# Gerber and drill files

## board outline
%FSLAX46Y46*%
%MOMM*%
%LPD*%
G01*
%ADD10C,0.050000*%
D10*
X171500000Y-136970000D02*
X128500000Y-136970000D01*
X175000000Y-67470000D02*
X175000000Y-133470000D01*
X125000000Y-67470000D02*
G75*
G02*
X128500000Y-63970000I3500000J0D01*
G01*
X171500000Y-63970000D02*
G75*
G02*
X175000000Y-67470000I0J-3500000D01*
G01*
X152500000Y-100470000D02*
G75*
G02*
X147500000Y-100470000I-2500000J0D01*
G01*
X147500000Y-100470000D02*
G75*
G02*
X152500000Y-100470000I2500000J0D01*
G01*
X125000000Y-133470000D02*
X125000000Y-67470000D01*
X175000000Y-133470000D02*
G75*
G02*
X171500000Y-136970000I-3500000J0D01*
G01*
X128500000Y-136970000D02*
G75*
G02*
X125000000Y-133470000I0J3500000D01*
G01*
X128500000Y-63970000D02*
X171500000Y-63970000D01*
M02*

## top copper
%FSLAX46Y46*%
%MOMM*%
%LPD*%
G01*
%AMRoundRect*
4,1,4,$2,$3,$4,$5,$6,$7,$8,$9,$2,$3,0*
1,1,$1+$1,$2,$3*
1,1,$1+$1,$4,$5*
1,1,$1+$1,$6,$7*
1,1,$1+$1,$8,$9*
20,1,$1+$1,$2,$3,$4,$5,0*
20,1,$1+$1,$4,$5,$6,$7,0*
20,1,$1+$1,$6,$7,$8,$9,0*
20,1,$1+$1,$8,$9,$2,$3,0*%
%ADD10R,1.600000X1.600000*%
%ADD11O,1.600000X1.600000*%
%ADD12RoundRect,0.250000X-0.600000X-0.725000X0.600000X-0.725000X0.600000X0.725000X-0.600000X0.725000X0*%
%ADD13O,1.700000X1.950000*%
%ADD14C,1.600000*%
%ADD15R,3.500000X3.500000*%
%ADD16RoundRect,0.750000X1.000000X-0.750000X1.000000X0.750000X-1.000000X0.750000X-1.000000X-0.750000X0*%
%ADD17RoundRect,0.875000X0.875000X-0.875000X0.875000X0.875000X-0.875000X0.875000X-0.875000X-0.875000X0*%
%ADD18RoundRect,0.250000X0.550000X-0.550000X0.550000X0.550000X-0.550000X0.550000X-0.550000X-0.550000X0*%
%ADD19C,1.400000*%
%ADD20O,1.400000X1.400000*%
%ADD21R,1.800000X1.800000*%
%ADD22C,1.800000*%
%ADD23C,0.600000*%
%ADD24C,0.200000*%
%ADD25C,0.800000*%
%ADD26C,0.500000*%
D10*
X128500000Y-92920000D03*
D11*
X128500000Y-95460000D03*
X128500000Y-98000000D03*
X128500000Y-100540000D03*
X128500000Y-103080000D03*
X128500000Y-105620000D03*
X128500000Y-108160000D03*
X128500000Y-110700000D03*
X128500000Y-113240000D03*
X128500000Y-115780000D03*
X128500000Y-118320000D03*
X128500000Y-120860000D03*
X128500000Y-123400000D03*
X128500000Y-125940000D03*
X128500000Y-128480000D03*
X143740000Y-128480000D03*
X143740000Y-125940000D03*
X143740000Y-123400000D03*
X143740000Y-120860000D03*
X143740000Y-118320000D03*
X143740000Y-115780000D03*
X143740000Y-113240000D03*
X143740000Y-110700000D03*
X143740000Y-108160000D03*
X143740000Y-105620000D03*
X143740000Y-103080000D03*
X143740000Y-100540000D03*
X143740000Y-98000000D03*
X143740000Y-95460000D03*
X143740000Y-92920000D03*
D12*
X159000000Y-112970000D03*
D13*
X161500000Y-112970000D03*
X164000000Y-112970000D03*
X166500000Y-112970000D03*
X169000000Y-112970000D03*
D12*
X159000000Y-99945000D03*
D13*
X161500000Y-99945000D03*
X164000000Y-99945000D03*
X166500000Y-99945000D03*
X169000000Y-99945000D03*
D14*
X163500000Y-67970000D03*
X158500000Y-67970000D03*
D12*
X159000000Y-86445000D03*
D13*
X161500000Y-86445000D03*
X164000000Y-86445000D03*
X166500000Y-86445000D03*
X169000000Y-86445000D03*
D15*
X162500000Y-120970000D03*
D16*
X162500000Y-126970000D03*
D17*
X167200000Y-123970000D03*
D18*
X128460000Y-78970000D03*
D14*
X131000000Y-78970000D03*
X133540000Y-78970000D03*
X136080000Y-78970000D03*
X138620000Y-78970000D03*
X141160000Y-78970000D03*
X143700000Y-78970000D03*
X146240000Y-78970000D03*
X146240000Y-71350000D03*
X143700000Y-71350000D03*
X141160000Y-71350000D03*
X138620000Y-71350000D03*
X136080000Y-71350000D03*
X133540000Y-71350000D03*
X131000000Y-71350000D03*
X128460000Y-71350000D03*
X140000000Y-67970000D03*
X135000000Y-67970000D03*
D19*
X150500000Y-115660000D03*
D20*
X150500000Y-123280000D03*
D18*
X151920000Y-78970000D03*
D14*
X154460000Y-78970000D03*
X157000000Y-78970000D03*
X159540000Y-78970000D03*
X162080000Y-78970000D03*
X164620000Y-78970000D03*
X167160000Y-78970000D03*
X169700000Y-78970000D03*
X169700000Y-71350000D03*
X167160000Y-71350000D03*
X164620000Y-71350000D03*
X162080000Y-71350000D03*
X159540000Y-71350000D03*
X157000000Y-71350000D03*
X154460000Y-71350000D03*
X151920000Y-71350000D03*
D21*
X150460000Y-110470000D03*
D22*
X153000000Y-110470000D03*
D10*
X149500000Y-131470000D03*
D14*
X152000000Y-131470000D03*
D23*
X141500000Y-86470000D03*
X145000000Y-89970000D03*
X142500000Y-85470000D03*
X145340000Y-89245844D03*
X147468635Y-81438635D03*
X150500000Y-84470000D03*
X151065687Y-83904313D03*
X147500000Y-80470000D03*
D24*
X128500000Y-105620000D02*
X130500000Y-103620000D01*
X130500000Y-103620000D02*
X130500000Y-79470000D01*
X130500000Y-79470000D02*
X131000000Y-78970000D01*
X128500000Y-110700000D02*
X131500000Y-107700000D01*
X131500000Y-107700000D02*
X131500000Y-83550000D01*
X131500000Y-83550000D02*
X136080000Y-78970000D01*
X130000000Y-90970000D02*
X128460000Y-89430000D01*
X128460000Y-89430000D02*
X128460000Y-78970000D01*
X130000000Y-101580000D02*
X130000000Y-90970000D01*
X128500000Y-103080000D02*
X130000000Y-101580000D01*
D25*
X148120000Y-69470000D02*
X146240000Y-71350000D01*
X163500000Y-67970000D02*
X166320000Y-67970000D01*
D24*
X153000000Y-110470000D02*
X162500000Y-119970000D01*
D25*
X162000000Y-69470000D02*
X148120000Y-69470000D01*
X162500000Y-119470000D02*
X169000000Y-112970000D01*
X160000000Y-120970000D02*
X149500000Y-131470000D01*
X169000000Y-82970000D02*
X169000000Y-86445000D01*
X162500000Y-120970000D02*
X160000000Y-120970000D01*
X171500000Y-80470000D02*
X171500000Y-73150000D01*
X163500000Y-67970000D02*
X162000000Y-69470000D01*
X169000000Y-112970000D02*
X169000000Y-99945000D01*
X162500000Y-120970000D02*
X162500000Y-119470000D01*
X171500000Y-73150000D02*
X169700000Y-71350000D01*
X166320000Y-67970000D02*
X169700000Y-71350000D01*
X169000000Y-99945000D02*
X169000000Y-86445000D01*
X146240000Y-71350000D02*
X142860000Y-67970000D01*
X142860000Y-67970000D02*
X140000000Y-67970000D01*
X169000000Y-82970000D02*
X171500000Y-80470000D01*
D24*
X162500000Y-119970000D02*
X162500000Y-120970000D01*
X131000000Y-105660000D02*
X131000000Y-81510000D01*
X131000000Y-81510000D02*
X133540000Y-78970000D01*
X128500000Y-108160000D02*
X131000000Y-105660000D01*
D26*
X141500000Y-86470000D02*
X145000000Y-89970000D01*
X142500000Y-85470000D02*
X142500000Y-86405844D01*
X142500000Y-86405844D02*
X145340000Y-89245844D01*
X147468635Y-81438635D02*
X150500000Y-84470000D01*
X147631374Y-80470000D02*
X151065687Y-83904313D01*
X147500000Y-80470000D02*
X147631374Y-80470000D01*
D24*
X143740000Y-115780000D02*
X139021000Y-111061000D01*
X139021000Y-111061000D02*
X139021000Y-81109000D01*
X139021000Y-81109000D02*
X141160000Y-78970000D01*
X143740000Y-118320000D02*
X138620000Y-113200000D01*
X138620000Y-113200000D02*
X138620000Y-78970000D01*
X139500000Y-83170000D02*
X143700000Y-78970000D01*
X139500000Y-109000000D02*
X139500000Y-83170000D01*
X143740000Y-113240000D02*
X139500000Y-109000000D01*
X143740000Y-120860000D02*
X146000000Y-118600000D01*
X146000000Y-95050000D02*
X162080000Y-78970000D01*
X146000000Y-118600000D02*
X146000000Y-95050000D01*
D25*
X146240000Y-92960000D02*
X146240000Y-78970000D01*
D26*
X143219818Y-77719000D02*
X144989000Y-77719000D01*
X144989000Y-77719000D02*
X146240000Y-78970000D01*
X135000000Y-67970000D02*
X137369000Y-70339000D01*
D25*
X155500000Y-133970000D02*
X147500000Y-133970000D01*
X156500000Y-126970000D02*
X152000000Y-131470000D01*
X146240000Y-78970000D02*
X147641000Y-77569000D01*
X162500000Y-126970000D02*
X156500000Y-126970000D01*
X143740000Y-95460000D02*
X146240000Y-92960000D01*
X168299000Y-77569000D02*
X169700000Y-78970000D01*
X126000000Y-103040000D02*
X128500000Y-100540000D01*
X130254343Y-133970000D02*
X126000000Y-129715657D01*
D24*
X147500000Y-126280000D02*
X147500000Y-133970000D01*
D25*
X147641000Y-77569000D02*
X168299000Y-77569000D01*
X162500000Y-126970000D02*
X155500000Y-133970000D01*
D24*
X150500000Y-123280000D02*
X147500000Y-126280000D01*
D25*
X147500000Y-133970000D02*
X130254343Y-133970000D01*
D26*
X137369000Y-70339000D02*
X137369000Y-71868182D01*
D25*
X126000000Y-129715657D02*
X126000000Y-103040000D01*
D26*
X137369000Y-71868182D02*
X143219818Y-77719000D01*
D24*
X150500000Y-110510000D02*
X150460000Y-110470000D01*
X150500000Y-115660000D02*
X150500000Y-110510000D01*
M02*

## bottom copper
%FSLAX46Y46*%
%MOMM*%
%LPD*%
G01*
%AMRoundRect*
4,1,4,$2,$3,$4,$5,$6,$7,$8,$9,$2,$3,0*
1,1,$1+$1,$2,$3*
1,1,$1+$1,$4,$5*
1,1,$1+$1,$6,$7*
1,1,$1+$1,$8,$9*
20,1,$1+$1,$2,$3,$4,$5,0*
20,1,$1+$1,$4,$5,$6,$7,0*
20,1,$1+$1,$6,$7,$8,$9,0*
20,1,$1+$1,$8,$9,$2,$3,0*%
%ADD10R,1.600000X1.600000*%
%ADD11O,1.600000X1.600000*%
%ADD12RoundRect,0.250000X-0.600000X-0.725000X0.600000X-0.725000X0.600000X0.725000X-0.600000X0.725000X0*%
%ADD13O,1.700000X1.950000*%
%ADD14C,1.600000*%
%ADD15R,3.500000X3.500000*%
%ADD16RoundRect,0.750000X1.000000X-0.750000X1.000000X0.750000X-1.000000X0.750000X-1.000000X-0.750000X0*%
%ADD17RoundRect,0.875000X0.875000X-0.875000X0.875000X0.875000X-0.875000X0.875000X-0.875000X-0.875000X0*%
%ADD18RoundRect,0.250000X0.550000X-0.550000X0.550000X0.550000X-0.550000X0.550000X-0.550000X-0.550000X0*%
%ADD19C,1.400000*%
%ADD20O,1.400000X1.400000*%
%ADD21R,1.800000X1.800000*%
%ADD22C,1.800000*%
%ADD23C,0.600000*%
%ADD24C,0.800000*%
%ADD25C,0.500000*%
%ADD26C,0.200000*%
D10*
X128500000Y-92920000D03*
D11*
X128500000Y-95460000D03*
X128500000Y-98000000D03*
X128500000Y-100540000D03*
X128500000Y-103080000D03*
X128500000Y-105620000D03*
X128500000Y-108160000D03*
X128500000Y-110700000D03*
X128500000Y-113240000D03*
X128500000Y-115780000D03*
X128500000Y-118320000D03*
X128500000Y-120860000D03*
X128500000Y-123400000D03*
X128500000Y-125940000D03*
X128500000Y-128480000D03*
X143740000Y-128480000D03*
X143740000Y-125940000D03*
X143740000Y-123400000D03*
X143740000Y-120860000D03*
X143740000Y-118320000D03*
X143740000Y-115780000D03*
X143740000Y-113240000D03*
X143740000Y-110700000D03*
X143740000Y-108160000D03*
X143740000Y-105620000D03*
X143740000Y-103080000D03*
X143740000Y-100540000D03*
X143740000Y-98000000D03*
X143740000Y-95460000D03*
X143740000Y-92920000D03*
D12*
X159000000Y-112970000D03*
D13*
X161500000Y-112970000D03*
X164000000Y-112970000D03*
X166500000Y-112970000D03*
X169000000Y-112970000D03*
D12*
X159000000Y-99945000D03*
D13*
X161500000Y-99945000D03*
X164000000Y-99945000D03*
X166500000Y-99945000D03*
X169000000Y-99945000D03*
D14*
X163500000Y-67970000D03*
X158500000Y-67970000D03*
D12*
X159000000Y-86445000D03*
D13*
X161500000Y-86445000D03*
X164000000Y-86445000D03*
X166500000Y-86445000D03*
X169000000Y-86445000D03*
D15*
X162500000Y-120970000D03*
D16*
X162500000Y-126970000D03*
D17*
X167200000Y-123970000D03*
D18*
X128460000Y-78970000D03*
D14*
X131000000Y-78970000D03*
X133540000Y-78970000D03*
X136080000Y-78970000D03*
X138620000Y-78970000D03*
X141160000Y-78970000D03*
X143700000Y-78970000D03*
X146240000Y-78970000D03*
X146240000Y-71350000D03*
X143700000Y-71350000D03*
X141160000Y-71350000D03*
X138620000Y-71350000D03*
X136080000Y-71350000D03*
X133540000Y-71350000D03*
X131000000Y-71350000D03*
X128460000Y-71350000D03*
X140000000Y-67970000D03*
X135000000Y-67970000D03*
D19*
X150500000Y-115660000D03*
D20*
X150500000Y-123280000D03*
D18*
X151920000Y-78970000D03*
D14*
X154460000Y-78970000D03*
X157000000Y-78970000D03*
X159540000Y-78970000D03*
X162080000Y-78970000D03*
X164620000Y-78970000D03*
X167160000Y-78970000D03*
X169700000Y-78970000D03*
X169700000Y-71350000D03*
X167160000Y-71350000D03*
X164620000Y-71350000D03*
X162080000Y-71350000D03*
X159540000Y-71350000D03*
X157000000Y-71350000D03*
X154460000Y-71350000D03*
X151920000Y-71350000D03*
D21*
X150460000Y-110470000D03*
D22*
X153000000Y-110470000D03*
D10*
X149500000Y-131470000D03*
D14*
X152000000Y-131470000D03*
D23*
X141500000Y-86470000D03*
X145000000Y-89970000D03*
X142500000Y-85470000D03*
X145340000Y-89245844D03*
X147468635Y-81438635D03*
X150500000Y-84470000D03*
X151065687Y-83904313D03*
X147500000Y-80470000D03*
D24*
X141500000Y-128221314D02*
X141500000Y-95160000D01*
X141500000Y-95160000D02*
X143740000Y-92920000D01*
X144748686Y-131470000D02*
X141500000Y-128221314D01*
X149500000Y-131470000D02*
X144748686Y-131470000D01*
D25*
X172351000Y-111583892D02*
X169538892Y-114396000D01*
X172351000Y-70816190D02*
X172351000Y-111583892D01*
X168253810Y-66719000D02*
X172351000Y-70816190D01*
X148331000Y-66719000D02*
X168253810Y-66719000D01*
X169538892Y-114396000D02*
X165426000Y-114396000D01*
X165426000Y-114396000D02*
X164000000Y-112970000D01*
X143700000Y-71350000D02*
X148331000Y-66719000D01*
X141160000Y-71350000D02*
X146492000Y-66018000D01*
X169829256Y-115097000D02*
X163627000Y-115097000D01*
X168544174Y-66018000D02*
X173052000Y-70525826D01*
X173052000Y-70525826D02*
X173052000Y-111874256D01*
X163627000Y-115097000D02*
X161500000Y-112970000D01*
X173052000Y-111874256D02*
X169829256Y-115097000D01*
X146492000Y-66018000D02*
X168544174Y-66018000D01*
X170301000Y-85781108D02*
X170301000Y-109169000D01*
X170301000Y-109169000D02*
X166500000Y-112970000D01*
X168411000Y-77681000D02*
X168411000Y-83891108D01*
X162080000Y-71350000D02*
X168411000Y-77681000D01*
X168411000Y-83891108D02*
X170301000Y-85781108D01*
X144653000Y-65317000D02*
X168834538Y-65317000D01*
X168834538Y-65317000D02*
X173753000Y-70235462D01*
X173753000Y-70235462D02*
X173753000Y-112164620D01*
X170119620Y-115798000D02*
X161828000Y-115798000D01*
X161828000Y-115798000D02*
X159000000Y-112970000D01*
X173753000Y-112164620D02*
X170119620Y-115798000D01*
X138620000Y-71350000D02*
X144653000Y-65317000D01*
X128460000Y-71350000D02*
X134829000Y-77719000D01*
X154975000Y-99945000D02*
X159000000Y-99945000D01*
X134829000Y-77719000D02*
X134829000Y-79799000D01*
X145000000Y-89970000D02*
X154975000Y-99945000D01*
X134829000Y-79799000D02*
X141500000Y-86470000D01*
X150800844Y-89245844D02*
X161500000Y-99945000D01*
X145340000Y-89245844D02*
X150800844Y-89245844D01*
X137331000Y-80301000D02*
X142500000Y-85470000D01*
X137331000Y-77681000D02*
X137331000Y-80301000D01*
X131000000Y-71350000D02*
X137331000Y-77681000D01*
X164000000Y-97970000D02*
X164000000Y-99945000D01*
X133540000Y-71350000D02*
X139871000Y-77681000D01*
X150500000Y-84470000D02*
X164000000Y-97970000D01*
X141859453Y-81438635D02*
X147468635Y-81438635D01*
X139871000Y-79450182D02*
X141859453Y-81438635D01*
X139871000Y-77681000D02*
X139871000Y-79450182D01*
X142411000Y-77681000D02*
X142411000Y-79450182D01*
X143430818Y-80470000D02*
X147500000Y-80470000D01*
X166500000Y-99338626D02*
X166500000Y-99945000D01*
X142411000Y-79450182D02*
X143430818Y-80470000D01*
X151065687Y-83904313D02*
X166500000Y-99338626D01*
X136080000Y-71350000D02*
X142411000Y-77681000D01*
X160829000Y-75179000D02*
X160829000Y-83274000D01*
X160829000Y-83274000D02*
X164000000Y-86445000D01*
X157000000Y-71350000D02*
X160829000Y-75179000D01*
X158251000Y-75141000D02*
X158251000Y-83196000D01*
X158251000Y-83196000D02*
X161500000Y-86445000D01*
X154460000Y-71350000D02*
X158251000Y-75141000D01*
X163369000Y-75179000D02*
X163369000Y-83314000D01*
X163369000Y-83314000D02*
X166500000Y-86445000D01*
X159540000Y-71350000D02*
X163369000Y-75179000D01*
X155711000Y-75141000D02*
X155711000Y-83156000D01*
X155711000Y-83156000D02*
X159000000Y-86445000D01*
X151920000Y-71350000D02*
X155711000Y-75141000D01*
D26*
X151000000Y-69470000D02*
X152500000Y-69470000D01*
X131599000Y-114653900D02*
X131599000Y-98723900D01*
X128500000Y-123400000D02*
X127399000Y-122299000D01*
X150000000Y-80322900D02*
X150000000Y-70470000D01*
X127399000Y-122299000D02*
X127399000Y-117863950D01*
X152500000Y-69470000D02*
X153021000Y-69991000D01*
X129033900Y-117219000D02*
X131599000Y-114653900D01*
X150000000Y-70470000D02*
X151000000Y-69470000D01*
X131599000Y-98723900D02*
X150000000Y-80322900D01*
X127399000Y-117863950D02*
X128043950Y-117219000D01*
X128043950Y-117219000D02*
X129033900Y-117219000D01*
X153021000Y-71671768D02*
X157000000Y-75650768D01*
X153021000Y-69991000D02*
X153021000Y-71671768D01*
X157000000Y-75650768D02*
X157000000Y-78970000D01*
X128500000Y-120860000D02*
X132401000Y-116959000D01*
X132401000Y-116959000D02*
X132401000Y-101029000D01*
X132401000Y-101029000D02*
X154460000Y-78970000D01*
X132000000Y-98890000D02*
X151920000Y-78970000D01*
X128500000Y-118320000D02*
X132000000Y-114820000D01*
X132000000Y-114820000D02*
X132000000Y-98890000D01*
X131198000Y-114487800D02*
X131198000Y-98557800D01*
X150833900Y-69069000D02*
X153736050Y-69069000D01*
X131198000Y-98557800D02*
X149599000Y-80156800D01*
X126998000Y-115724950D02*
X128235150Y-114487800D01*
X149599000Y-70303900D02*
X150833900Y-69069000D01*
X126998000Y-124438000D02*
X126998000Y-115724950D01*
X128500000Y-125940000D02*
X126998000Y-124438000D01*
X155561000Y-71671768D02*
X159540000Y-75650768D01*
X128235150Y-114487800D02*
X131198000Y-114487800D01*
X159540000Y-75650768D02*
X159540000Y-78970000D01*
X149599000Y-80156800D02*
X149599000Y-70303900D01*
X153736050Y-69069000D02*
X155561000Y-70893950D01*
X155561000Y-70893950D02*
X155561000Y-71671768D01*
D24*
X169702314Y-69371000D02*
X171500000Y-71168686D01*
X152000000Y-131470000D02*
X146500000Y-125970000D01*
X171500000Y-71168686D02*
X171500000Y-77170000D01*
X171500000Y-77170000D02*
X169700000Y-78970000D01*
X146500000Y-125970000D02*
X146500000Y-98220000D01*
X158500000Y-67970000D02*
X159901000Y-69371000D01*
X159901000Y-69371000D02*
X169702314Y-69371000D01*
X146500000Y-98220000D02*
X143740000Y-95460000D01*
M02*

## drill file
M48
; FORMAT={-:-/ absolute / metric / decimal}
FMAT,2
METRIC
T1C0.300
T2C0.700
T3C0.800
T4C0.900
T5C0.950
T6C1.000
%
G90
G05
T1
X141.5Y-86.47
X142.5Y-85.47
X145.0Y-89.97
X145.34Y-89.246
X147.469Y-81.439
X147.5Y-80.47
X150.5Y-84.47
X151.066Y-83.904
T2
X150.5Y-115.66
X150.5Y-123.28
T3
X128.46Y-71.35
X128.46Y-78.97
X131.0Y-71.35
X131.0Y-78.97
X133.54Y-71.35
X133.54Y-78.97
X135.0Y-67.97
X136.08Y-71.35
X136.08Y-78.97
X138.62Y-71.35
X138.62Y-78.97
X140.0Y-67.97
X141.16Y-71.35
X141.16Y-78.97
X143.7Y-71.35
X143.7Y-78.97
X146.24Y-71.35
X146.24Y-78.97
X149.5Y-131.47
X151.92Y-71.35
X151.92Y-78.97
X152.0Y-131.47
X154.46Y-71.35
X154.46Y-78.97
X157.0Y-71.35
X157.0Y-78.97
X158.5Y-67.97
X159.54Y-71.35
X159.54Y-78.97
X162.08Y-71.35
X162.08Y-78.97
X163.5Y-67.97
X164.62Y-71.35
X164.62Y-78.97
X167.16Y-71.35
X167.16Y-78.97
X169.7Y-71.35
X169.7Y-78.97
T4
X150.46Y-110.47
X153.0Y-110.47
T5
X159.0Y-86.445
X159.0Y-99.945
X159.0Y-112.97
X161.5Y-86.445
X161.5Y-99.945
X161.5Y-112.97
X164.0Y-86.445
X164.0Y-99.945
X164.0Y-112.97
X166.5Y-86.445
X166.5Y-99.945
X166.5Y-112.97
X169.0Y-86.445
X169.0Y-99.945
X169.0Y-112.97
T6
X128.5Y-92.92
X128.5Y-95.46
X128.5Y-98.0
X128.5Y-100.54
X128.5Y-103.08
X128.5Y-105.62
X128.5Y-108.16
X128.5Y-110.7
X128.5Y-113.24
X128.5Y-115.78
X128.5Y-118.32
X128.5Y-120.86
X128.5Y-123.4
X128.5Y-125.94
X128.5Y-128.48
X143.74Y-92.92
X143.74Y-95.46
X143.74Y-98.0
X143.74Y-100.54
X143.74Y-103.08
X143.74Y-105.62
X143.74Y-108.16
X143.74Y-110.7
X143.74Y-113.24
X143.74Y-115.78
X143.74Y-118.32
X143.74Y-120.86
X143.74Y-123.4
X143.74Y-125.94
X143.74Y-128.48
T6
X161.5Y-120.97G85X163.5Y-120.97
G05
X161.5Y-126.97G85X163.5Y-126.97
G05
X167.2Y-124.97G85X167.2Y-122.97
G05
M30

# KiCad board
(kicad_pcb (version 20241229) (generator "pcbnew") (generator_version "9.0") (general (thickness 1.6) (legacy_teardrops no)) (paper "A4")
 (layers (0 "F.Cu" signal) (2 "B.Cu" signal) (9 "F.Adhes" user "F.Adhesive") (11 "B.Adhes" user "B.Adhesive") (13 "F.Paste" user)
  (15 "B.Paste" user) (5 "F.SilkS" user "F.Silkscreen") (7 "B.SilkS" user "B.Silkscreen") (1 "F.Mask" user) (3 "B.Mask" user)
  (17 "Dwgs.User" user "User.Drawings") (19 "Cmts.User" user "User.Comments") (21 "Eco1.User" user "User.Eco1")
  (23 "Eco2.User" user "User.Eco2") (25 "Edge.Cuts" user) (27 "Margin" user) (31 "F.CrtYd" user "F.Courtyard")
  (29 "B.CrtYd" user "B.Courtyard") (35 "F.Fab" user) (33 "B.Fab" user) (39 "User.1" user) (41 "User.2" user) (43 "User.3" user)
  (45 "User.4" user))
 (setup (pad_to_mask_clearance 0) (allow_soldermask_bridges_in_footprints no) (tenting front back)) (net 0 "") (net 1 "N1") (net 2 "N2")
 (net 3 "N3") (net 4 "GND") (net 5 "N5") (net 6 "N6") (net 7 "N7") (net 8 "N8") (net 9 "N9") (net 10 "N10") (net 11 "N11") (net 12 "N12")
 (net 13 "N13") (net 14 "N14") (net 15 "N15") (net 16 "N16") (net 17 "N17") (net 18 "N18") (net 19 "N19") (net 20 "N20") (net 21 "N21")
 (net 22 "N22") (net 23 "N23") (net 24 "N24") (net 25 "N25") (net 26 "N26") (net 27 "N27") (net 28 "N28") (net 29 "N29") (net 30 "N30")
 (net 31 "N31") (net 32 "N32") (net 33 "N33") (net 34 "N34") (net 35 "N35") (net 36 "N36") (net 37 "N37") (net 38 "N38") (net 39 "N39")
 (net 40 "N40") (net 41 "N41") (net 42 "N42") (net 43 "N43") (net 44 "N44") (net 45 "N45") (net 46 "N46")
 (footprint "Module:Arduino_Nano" (layer "F.Cu") (at 128.5 92.92)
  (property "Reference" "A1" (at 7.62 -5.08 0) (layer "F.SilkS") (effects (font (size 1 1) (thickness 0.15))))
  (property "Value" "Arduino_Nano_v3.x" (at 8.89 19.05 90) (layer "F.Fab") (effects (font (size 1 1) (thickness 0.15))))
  (pad "1" thru_hole rect (at 0 0) (size 1.6 1.6) (drill 1) (layers "*.Cu" "*.Mask") (remove_unused_layers no) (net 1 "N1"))
  (pad "2" thru_hole oval (at 0 2.54) (size 1.6 1.6) (drill 1) (layers "*.Cu" "*.Mask") (remove_unused_layers no) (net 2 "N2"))
  (pad "3" thru_hole oval (at 0 5.08) (size 1.6 1.6) (drill 1) (layers "*.Cu" "*.Mask") (remove_unused_layers no) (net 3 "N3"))
  (pad "4" thru_hole oval (at 0 7.62) (size 1.6 1.6) (drill 1) (layers "*.Cu" "*.Mask") (remove_unused_layers no) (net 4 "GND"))
  (pad "5" thru_hole oval (at 0 10.16) (size 1.6 1.6) (drill 1) (layers "*.Cu" "*.Mask") (remove_unused_layers no) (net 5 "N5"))
  (pad "6" thru_hole oval (at 0 12.7) (size 1.6 1.6) (drill 1) (layers "*.Cu" "*.Mask") (remove_unused_layers no) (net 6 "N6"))
  (pad "7" thru_hole oval (at 0 15.24) (size 1.6 1.6) (drill 1) (layers "*.Cu" "*.Mask") (remove_unused_layers no) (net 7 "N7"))
  (pad "8" thru_hole oval (at 0 17.78) (size 1.6 1.6) (drill 1) (layers "*.Cu" "*.Mask") (remove_unused_layers no) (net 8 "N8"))
  (pad "9" thru_hole oval (at 0 20.32) (size 1.6 1.6) (drill 1) (layers "*.Cu" "*.Mask") (remove_unused_layers no) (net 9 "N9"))
  (pad "10" thru_hole oval (at 0 22.86) (size 1.6 1.6) (drill 1) (layers "*.Cu" "*.Mask") (remove_unused_layers no) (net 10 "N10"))
  (pad "11" thru_hole oval (at 0 25.4) (size 1.6 1.6) (drill 1) (layers "*.Cu" "*.Mask") (remove_unused_layers no) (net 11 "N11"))
  (pad "12" thru_hole oval (at 0 27.94) (size 1.6 1.6) (drill 1) (layers "*.Cu" "*.Mask") (remove_unused_layers no) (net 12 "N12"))
  (pad "13" thru_hole oval (at 0 30.48) (size 1.6 1.6) (drill 1) (layers "*.Cu" "*.Mask") (remove_unused_layers no) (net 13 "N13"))
  (pad "14" thru_hole oval (at 0 33.02) (size 1.6 1.6) (drill 1) (layers "*.Cu" "*.Mask") (remove_unused_layers no) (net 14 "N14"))
  (pad "15" thru_hole oval (at 0 35.56) (size 1.6 1.6) (drill 1) (layers "*.Cu" "*.Mask") (remove_unused_layers no) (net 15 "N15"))
  (pad "16" thru_hole oval (at 15.24 35.56) (size 1.6 1.6) (drill 1) (layers "*.Cu" "*.Mask") (remove_unused_layers no) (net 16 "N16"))
  (pad "17" thru_hole oval (at 15.24 33.02) (size 1.6 1.6) (drill 1) (layers "*.Cu" "*.Mask") (remove_unused_layers no) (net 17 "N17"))
  (pad "18" thru_hole oval (at 15.24 30.48) (size 1.6 1.6) (drill 1) (layers "*.Cu" "*.Mask") (remove_unused_layers no) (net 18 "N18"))
  (pad "19" thru_hole oval (at 15.24 27.94) (size 1.6 1.6) (drill 1) (layers "*.Cu" "*.Mask") (remove_unused_layers no) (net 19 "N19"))
  (pad "20" thru_hole oval (at 15.24 25.4) (size 1.6 1.6) (drill 1) (layers "*.Cu" "*.Mask") (remove_unused_layers no) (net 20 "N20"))
  (pad "21" thru_hole oval (at 15.24 22.86) (size 1.6 1.6) (drill 1) (layers "*.Cu" "*.Mask") (remove_unused_layers no) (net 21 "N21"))
  (pad "22" thru_hole oval (at 15.24 20.32) (size 1.6 1.6) (drill 1) (layers "*.Cu" "*.Mask") (remove_unused_layers no) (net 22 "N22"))
  (pad "23" thru_hole oval (at 15.24 17.78) (size 1.6 1.6) (drill 1) (layers "*.Cu" "*.Mask") (remove_unused_layers no) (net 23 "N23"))
  (pad "24" thru_hole oval (at 15.24 15.24) (size 1.6 1.6) (drill 1) (layers "*.Cu" "*.Mask") (remove_unused_layers no) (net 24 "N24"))
  (pad "25" thru_hole oval (at 15.24 12.7) (size 1.6 1.6) (drill 1) (layers "*.Cu" "*.Mask") (remove_unused_layers no) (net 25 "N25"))
  (pad "26" thru_hole oval (at 15.24 10.16) (size 1.6 1.6) (drill 1) (layers "*.Cu" "*.Mask") (remove_unused_layers no) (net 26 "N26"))
  (pad "27" thru_hole oval (at 15.24 7.62) (size 1.6 1.6) (drill 1) (layers "*.Cu" "*.Mask") (remove_unused_layers no) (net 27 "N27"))
  (pad "28" thru_hole oval (at 15.24 5.08) (size 1.6 1.6) (drill 1) (layers "*.Cu" "*.Mask") (remove_unused_layers no) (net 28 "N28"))
  (pad "29" thru_hole oval (at 15.24 2.54) (size 1.6 1.6) (drill 1) (layers "*.Cu" "*.Mask") (remove_unused_layers no) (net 4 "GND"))
  (pad "30" thru_hole oval (at 15.24 0) (size 1.6 1.6) (drill 1) (layers "*.Cu" "*.Mask") (remove_unused_layers no) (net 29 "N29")))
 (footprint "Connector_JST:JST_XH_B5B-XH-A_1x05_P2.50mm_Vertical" (layer "F.Cu") (at 159 112.97)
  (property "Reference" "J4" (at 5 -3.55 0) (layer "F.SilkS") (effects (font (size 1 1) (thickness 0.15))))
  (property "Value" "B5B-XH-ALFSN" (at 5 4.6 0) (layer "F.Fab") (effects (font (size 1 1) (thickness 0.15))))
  (pad "1" thru_hole roundrect (at 0 0) (size 1.7 1.95) (drill 0.95) (layers "*.Cu" "*.Mask") (remove_unused_layers no)
   (roundrect_rratio 0.147059) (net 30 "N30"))
  (pad "2" thru_hole oval (at 2.5 0) (size 1.7 1.95) (drill 0.95) (layers "*.Cu" "*.Mask") (remove_unused_layers no) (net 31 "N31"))
  (pad "3" thru_hole oval (at 5 0) (size 1.7 1.95) (drill 0.95) (layers "*.Cu" "*.Mask") (remove_unused_layers no) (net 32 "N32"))
  (pad "4" thru_hole oval (at 7.5 0) (size 1.7 1.95) (drill 0.95) (layers "*.Cu" "*.Mask") (remove_unused_layers no) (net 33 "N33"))
  (pad "5" thru_hole oval (at 10 0) (size 1.7 1.95) (drill 0.95) (layers "*.Cu" "*.Mask") (remove_unused_layers no) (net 29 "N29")))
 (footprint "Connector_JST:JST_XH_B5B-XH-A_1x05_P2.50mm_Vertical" (layer "F.Cu") (at 159 99.945)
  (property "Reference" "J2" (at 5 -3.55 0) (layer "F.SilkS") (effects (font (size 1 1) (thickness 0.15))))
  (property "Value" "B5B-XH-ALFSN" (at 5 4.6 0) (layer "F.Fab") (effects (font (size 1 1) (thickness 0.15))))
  (pad "1" thru_hole roundrect (at 0 0) (size 1.7 1.95) (drill 0.95) (layers "*.Cu" "*.Mask") (remove_unused_layers no)
   (roundrect_rratio 0.147059) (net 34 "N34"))
  (pad "2" thru_hole oval (at 2.5 0) (size 1.7 1.95) (drill 0.95) (layers "*.Cu" "*.Mask") (remove_unused_layers no) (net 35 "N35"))
  (pad "3" thru_hole oval (at 5 0) (size 1.7 1.95) (drill 0.95) (layers "*.Cu" "*.Mask") (remove_unused_layers no) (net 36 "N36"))
  (pad "4" thru_hole oval (at 7.5 0) (size 1.7 1.95) (drill 0.95) (layers "*.Cu" "*.Mask") (remove_unused_layers no) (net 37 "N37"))
  (pad "5" thru_hole oval (at 10 0) (size 1.7 1.95) (drill 0.95) (layers "*.Cu" "*.Mask") (remove_unused_layers no) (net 29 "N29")))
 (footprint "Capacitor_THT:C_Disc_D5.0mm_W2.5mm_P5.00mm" (layer "F.Cu") (at 163.5 67.97 180)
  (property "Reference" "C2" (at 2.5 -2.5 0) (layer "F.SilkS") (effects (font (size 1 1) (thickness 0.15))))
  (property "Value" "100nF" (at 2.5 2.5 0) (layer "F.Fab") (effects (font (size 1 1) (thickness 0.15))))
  (pad "1" thru_hole circle (at 0 0 180) (size 1.6 1.6) (drill 0.8) (layers "*.Cu" "*.Mask") (remove_unused_layers no) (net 29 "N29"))
  (pad "2" thru_hole circle (at 5 0 180) (size 1.6 1.6) (drill 0.8) (layers "*.Cu" "*.Mask") (remove_unused_layers no) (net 4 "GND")))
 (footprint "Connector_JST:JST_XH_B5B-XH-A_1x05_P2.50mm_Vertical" (layer "F.Cu") (at 159 86.445)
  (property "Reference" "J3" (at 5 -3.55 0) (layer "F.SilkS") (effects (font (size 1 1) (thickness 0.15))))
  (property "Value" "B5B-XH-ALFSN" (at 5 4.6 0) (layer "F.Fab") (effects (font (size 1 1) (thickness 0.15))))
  (pad "1" thru_hole roundrect (at 0 0) (size 1.7 1.95) (drill 0.95) (layers "*.Cu" "*.Mask") (remove_unused_layers no)
   (roundrect_rratio 0.147059) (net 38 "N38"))
  (pad "2" thru_hole oval (at 2.5 0) (size 1.7 1.95) (drill 0.95) (layers "*.Cu" "*.Mask") (remove_unused_layers no) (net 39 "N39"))
  (pad "3" thru_hole oval (at 5 0) (size 1.7 1.95) (drill 0.95) (layers "*.Cu" "*.Mask") (remove_unused_layers no) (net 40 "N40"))
  (pad "4" thru_hole oval (at 7.5 0) (size 1.7 1.95) (drill 0.95) (layers "*.Cu" "*.Mask") (remove_unused_layers no) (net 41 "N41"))
  (pad "5" thru_hole oval (at 10 0) (size 1.7 1.95) (drill 0.95) (layers "*.Cu" "*.Mask") (remove_unused_layers no) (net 29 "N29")))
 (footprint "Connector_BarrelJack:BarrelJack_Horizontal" (layer "F.Cu") (at 162.5 120.97 90)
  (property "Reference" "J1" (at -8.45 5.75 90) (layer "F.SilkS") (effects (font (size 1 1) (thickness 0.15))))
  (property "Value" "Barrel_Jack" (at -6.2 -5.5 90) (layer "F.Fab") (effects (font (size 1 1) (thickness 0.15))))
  (pad "1" thru_hole rect (at 0 0 90) (size 3.5 3.5) (drill oval 1 3) (layers "*.Cu" "*.Mask") (remove_unused_layers no) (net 29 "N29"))
  (pad "2" thru_hole roundrect (at -6 0 90) (size 3 3.5) (drill oval 1 3) (layers "*.Cu" "*.Mask") (remove_unused_layers no)
   (roundrect_rratio 0.25) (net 4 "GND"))
  (pad "3" thru_hole roundrect (at -3 4.7 90) (size 3.5 3.5) (drill oval 3 1) (layers "*.Cu" "*.Mask") (remove_unused_layers no)
   (roundrect_rratio 0.25)))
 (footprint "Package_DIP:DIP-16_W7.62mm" (layer "F.Cu") (at 128.46 78.97 90)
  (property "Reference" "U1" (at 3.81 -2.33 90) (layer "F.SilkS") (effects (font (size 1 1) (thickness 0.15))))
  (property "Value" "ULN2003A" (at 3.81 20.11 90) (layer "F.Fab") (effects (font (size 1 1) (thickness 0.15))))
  (pad "1" thru_hole roundrect (at 0 0 90) (size 1.6 1.6) (drill 0.8) (layers "*.Cu" "*.Mask") (remove_unused_layers no)
   (roundrect_rratio 0.15625) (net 5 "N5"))
  (pad "2" thru_hole circle (at 0 2.54 90) (size 1.6 1.6) (drill 0.8) (layers "*.Cu" "*.Mask") (remove_unused_layers no) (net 6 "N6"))
  (pad "3" thru_hole circle (at 0 5.08 90) (size 1.6 1.6) (drill 0.8) (layers "*.Cu" "*.Mask") (remove_unused_layers no) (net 7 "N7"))
  (pad "4" thru_hole circle (at 0 7.62 90) (size 1.6 1.6) (drill 0.8) (layers "*.Cu" "*.Mask") (remove_unused_layers no) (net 8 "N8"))
  (pad "5" thru_hole circle (at 0 10.16 90) (size 1.6 1.6) (drill 0.8) (layers "*.Cu" "*.Mask") (remove_unused_layers no) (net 20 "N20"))
  (pad "6" thru_hole circle (at 0 12.7 90) (size 1.6 1.6) (drill 0.8) (layers "*.Cu" "*.Mask") (remove_unused_layers no) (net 21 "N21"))
  (pad "7" thru_hole circle (at 0 15.24 90) (size 1.6 1.6) (drill 0.8) (layers "*.Cu" "*.Mask") (remove_unused_layers no) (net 22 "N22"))
  (pad "8" thru_hole circle (at 0 17.78 90) (size 1.6 1.6) (drill 0.8) (layers "*.Cu" "*.Mask") (remove_unused_layers no) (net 4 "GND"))
  (pad "9" thru_hole circle (at 7.62 17.78 90) (size 1.6 1.6) (drill 0.8) (layers "*.Cu" "*.Mask") (remove_unused_layers no) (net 29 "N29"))
  (pad "10" thru_hole circle (at 7.62 15.24 90) (size 1.6 1.6) (drill 0.8) (layers "*.Cu" "*.Mask") (remove_unused_layers no) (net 32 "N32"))
  (pad "11" thru_hole circle (at 7.62 12.7 90) (size 1.6 1.6) (drill 0.8) (layers "*.Cu" "*.Mask") (remove_unused_layers no) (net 31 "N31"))
  (pad "12" thru_hole circle (at 7.62 10.16 90) (size 1.6 1.6) (drill 0.8) (layers "*.Cu" "*.Mask") (remove_unused_layers no) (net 30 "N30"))
  (pad "13" thru_hole circle (at 7.62 7.62 90) (size 1.6 1.6) (drill 0.8) (layers "*.Cu" "*.Mask") (remove_unused_layers no) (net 37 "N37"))
  (pad "14" thru_hole circle (at 7.62 5.08 90) (size 1.6 1.6) (drill 0.8) (layers "*.Cu" "*.Mask") (remove_unused_layers no) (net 36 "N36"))
  (pad "15" thru_hole circle (at 7.62 2.54 90) (size 1.6 1.6) (drill 0.8) (layers "*.Cu" "*.Mask") (remove_unused_layers no) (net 35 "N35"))
  (pad "16" thru_hole circle (at 7.62 0 90) (size 1.6 1.6) (drill 0.8) (layers "*.Cu" "*.Mask") (remove_unused_layers no) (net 34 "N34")))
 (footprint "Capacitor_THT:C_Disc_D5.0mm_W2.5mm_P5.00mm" (layer "F.Cu") (at 140 67.97 180)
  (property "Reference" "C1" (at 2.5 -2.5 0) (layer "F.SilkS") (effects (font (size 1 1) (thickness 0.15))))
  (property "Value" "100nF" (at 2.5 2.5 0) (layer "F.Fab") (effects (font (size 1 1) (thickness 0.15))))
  (pad "1" thru_hole circle (at 0 0 180) (size 1.6 1.6) (drill 0.8) (layers "*.Cu" "*.Mask") (remove_unused_layers no) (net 29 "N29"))
  (pad "2" thru_hole circle (at 5 0 180) (size 1.6 1.6) (drill 0.8) (layers "*.Cu" "*.Mask") (remove_unused_layers no) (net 4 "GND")))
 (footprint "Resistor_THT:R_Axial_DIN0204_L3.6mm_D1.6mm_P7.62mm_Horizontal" (layer "F.Cu") (at 150.5 115.66 -90)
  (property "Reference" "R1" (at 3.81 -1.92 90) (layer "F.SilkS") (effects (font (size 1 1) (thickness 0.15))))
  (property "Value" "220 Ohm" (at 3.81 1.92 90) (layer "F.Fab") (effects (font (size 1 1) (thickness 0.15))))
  (pad "1" thru_hole circle (at 0 0 270) (size 1.4 1.4) (drill 0.7) (layers "*.Cu" "*.Mask") (remove_unused_layers no) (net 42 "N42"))
  (pad "2" thru_hole oval (at 7.62 0 270) (size 1.4 1.4) (drill 0.7) (layers "*.Cu" "*.Mask") (remove_unused_layers no) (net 4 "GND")))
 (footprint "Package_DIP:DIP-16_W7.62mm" (layer "F.Cu") (at 151.92 78.97 90)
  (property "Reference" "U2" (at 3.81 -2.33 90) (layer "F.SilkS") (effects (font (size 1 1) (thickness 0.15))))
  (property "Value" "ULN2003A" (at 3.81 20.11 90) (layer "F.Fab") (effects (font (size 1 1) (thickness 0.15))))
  (pad "1" thru_hole roundrect (at 0 0 90) (size 1.6 1.6) (drill 0.8) (layers "*.Cu" "*.Mask") (remove_unused_layers no)
   (roundrect_rratio 0.15625) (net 11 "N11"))
  (pad "2" thru_hole circle (at 0 2.54 90) (size 1.6 1.6) (drill 0.8) (layers "*.Cu" "*.Mask") (remove_unused_layers no) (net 12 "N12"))
  (pad "3" thru_hole circle (at 0 5.08 90) (size 1.6 1.6) (drill 0.8) (layers "*.Cu" "*.Mask") (remove_unused_layers no) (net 13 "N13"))
  (pad "4" thru_hole circle (at 0 7.62 90) (size 1.6 1.6) (drill 0.8) (layers "*.Cu" "*.Mask") (remove_unused_layers no) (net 14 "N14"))
  (pad "5" thru_hole circle (at 0 10.16 90) (size 1.6 1.6) (drill 0.8) (layers "*.Cu" "*.Mask") (remove_unused_layers no) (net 19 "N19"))
  (pad "6" thru_hole circle (at 0 12.7 90) (size 1.6 1.6) (drill 0.8) (layers "*.Cu" "*.Mask") (remove_unused_layers no) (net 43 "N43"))
  (pad "7" thru_hole circle (at 0 15.24 90) (size 1.6 1.6) (drill 0.8) (layers "*.Cu" "*.Mask") (remove_unused_layers no) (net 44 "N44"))
  (pad "8" thru_hole circle (at 0 17.78 90) (size 1.6 1.6) (drill 0.8) (layers "*.Cu" "*.Mask") (remove_unused_layers no) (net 4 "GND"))
  (pad "9" thru_hole circle (at 7.62 17.78 90) (size 1.6 1.6) (drill 0.8) (layers "*.Cu" "*.Mask") (remove_unused_layers no) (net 29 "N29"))
  (pad "10" thru_hole circle (at 7.62 15.24 90) (size 1.6 1.6) (drill 0.8) (layers "*.Cu" "*.Mask") (remove_unused_layers no) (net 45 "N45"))
  (pad "11" thru_hole circle (at 7.62 12.7 90) (size 1.6 1.6) (drill 0.8) (layers "*.Cu" "*.Mask") (remove_unused_layers no) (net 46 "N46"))
  (pad "12" thru_hole circle (at 7.62 10.16 90) (size 1.6 1.6) (drill 0.8) (layers "*.Cu" "*.Mask") (remove_unused_layers no) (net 33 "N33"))
  (pad "13" thru_hole circle (at 7.62 7.62 90) (size 1.6 1.6) (drill 0.8) (layers "*.Cu" "*.Mask") (remove_unused_layers no) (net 41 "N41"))
  (pad "14" thru_hole circle (at 7.62 5.08 90) (size 1.6 1.6) (drill 0.8) (layers "*.Cu" "*.Mask") (remove_unused_layers no) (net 40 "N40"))
  (pad "15" thru_hole circle (at 7.62 2.54 90) (size 1.6 1.6) (drill 0.8) (layers "*.Cu" "*.Mask") (remove_unused_layers no) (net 39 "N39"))
  (pad "16" thru_hole circle (at 7.62 0 90) (size 1.6 1.6) (drill 0.8) (layers "*.Cu" "*.Mask") (remove_unused_layers no) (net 38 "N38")))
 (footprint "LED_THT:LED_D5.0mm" (layer "F.Cu") (at 150.46 110.47)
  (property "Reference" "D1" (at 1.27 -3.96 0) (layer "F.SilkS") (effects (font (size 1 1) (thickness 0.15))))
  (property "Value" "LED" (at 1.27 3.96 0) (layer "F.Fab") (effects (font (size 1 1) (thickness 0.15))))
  (pad "1" thru_hole rect (at 0 0) (size 1.8 1.8) (drill 0.9) (layers "*.Cu" "*.Mask") (remove_unused_layers no) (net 42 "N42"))
  (pad "2" thru_hole circle (at 2.54 0) (size 1.8 1.8) (drill 0.9) (layers "*.Cu" "*.Mask") (remove_unused_layers no) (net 29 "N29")))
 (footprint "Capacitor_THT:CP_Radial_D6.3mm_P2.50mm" (layer "F.Cu") (at 149.5 131.47)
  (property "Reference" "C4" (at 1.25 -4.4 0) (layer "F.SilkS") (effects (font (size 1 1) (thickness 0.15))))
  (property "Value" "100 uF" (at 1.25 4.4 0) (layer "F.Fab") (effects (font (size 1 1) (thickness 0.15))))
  (pad "1" thru_hole rect (at 0 0) (size 1.6 1.6) (drill 0.8) (layers "*.Cu" "*.Mask") (remove_unused_layers no) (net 29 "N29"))
  (pad "2" thru_hole circle (at 2.5 0) (size 1.6 1.6) (drill 0.8) (layers "*.Cu" "*.Mask") (remove_unused_layers no) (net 4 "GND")))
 (gr_line (start 171.5 136.97) (end 128.5 136.97) (stroke (width 0.05) (type default)) (layer "Edge.Cuts"))
 (gr_line (start 175 67.47) (end 175 133.47) (stroke (width 0.05) (type default)) (layer "Edge.Cuts"))
 (gr_arc (start 125 67.47) (mid 126.025126 64.995126) (end 128.5 63.97) (stroke (width 0.05) (type default)) (layer "Edge.Cuts"))
 (gr_arc (start 171.5 63.97) (mid 173.974874 64.995126) (end 175 67.47) (stroke (width 0.05) (type default)) (layer "Edge.Cuts"))
 (gr_circle (center 150 100.47) (end 152.5 100.47) (stroke (width 0.05) (type default)) (fill no) (layer "Edge.Cuts"))
 (gr_line (start 125 133.47) (end 125 67.47) (stroke (width 0.05) (type default)) (layer "Edge.Cuts"))
 (gr_arc (start 175 133.47) (mid 173.974874 135.944874) (end 171.5 136.97) (stroke (width 0.05) (type default)) (layer "Edge.Cuts"))
 (gr_arc (start 128.5 136.97) (mid 126.025126 135.944874) (end 125 133.47) (stroke (width 0.05) (type default)) (layer "Edge.Cuts"))
 (gr_line (start 128.5 63.97) (end 171.5 63.97) (stroke (width 0.05) (type default)) (layer "Edge.Cuts"))
 (segment (start 128.5 105.62) (end 130.5 103.62) (width 0.2) (layer "F.Cu") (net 6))
 (segment (start 130.5 103.62) (end 130.5 79.47) (width 0.2) (layer "F.Cu") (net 6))
 (segment (start 130.5 79.47) (end 131 78.97) (width 0.2) (layer "F.Cu") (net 6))
 (segment (start 128.5 110.7) (end 131.5 107.7) (width 0.2) (layer "F.Cu") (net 8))
 (segment (start 131.5 107.7) (end 131.5 83.55) (width 0.2) (layer "F.Cu") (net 8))
 (segment (start 131.5 83.55) (end 136.08 78.97) (width 0.2) (layer "F.Cu") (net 8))
 (segment (start 130 90.97) (end 128.46 89.43) (width 0.2) (layer "F.Cu") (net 5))
 (segment (start 128.46 89.43) (end 128.46 78.97) (width 0.2) (layer "F.Cu") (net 5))
 (segment (start 130 101.58) (end 130 90.97) (width 0.2) (layer "F.Cu") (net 5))
 (segment (start 128.5 103.08) (end 130 101.58) (width 0.2) (layer "F.Cu") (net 5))
 (segment (start 148.12 69.47) (end 146.24 71.35) (width 0.8) (layer "F.Cu") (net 29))
 (segment (start 163.5 67.97) (end 166.32 67.97) (width 0.8) (layer "F.Cu") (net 29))
 (segment (start 153 110.47) (end 162.5 119.97) (width 0.2) (layer "F.Cu") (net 29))
 (segment (start 162 69.47) (end 148.12 69.47) (width 0.8) (layer "F.Cu") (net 29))
 (segment (start 162.5 119.47) (end 169 112.97) (width 0.8) (layer "F.Cu") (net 29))
 (segment (start 160 120.97) (end 149.5 131.47) (width 0.8) (layer "F.Cu") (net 29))
 (segment (start 169 82.97) (end 169 86.445) (width 0.8) (layer "F.Cu") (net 29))
 (segment (start 162.5 120.97) (end 160 120.97) (width 0.8) (layer "F.Cu") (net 29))
 (segment (start 171.5 80.47) (end 171.5 73.15) (width 0.8) (layer "F.Cu") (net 29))
 (segment (start 163.5 67.97) (end 162 69.47) (width 0.8) (layer "F.Cu") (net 29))
 (segment (start 169 112.97) (end 169 99.945) (width 0.8) (layer "F.Cu") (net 29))
 (segment (start 162.5 120.97) (end 162.5 119.47) (width 0.8) (layer "F.Cu") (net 29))
 (segment (start 171.5 73.15) (end 169.7 71.35) (width 0.8) (layer "F.Cu") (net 29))
 (segment (start 166.32 67.97) (end 169.7 71.35) (width 0.8) (layer "F.Cu") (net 29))
 (segment (start 169 99.945) (end 169 86.445) (width 0.8) (layer "F.Cu") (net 29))
 (segment (start 146.24 71.35) (end 142.86 67.97) (width 0.8) (layer "F.Cu") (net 29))
 (segment (start 142.86 67.97) (end 140 67.97) (width 0.8) (layer "F.Cu") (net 29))
 (segment (start 169 82.97) (end 171.5 80.47) (width 0.8) (layer "F.Cu") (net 29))
 (segment (start 162.5 119.97) (end 162.5 120.97) (width 0.2) (layer "F.Cu") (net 29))
 (segment (start 141.5 128.221314) (end 141.5 95.16) (width 0.8) (layer "B.Cu") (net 29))
 (segment (start 141.5 95.16) (end 143.74 92.92) (width 0.8) (layer "B.Cu") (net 29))
 (segment (start 144.748686 131.47) (end 141.5 128.221314) (width 0.8) (layer "B.Cu") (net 29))
 (segment (start 149.5 131.47) (end 144.748686 131.47) (width 0.8) (layer "B.Cu") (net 29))
 (segment (start 131 105.66) (end 131 81.51) (width 0.2) (layer "F.Cu") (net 7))
 (segment (start 131 81.51) (end 133.54 78.97) (width 0.2) (layer "F.Cu") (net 7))
 (segment (start 128.5 108.16) (end 131 105.66) (width 0.2) (layer "F.Cu") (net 7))
 (segment (start 172.351 111.583892) (end 169.538892 114.396) (width 0.5) (layer "B.Cu") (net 32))
 (segment (start 172.351 70.81619) (end 172.351 111.583892) (width 0.5) (layer "B.Cu") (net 32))
 (segment (start 168.25381 66.719) (end 172.351 70.81619) (width 0.5) (layer "B.Cu") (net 32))
 (segment (start 148.331 66.719) (end 168.25381 66.719) (width 0.5) (layer "B.Cu") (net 32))
 (segment (start 169.538892 114.396) (end 165.426 114.396) (width 0.5) (layer "B.Cu") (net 32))
 (segment (start 165.426 114.396) (end 164 112.97) (width 0.5) (layer "B.Cu") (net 32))
 (segment (start 143.7 71.35) (end 148.331 66.719) (width 0.5) (layer "B.Cu") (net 32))
 (segment (start 141.16 71.35) (end 146.492 66.018) (width 0.5) (layer "B.Cu") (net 31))
 (segment (start 169.829256 115.097) (end 163.627 115.097) (width 0.5) (layer "B.Cu") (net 31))
 (segment (start 168.544174 66.018) (end 173.052 70.525826) (width 0.5) (layer "B.Cu") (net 31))
 (segment (start 173.052 70.525826) (end 173.052 111.874256) (width 0.5) (layer "B.Cu") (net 31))
 (segment (start 163.627 115.097) (end 161.5 112.97) (width 0.5) (layer "B.Cu") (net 31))
 (segment (start 173.052 111.874256) (end 169.829256 115.097) (width 0.5) (layer "B.Cu") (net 31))
 (segment (start 146.492 66.018) (end 168.544174 66.018) (width 0.5) (layer "B.Cu") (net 31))
 (segment (start 170.301 85.781108) (end 170.301 109.169) (width 0.5) (layer "B.Cu") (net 33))
 (segment (start 170.301 109.169) (end 166.5 112.97) (width 0.5) (layer "B.Cu") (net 33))
 (segment (start 168.411 77.681) (end 168.411 83.891108) (width 0.5) (layer "B.Cu") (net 33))
 (segment (start 162.08 71.35) (end 168.411 77.681) (width 0.5) (layer "B.Cu") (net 33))
 (segment (start 168.411 83.891108) (end 170.301 85.781108) (width 0.5) (layer "B.Cu") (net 33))
 (segment (start 144.653 65.317) (end 168.834538 65.317) (width 0.5) (layer "B.Cu") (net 30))
 (segment (start 168.834538 65.317) (end 173.753 70.235462) (width 0.5) (layer "B.Cu") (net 30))
 (segment (start 173.753 70.235462) (end 173.753 112.16462) (width 0.5) (layer "B.Cu") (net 30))
 (segment (start 170.11962 115.798) (end 161.828 115.798) (width 0.5) (layer "B.Cu") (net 30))
 (segment (start 161.828 115.798) (end 159 112.97) (width 0.5) (layer "B.Cu") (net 30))
 (segment (start 173.753 112.16462) (end 170.11962 115.798) (width 0.5) (layer "B.Cu") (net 30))
 (segment (start 138.62 71.35) (end 144.653 65.317) (width 0.5) (layer "B.Cu") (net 30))
 (segment (start 141.5 86.47) (end 145 89.97) (width 0.5) (layer "F.Cu") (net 34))
 (via (at 141.5 86.47) (size 0.6) (drill 0.3) (layers "F.Cu" "B.Cu") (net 34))
 (via (at 145 89.97) (size 0.6) (drill 0.3) (layers "F.Cu" "B.Cu") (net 34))
 (segment (start 128.46 71.35) (end 134.829 77.719) (width 0.5) (layer "B.Cu") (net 34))
 (segment (start 154.975 99.945) (end 159 99.945) (width 0.5) (layer "B.Cu") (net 34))
 (segment (start 134.829 77.719) (end 134.829 79.799) (width 0.5) (layer "B.Cu") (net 34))
 (segment (start 145 89.97) (end 154.975 99.945) (width 0.5) (layer "B.Cu") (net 34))
 (segment (start 134.829 79.799) (end 141.5 86.47) (width 0.5) (layer "B.Cu") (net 34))
 (segment (start 142.5 85.47) (end 142.5 86.405844) (width 0.5) (layer "F.Cu") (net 35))
 (segment (start 142.5 86.405844) (end 145.34 89.245844) (width 0.5) (layer "F.Cu") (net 35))
 (via (at 142.5 85.47) (size 0.6) (drill 0.3) (layers "F.Cu" "B.Cu") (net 35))
 (via (at 145.34 89.245844) (size 0.6) (drill 0.3) (layers "F.Cu" "B.Cu") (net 35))
 (segment (start 150.800844 89.245844) (end 161.5 99.945) (width 0.5) (layer "B.Cu") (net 35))
 (segment (start 145.34 89.245844) (end 150.800844 89.245844) (width 0.5) (layer "B.Cu") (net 35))
 (segment (start 137.331 80.301) (end 142.5 85.47) (width 0.5) (layer "B.Cu") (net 35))
 (segment (start 137.331 77.681) (end 137.331 80.301) (width 0.5) (layer "B.Cu") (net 35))
 (segment (start 131 71.35) (end 137.331 77.681) (width 0.5) (layer "B.Cu") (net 35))
 (segment (start 147.468635 81.438635) (end 150.5 84.47) (width 0.5) (layer "F.Cu") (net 36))
 (via (at 147.468635 81.438635) (size 0.6) (drill 0.3) (layers "F.Cu" "B.Cu") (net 36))
 (via (at 150.5 84.47) (size 0.6) (drill 0.3) (layers "F.Cu" "B.Cu") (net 36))
 (segment (start 164 97.97) (end 164 99.945) (width 0.5) (layer "B.Cu") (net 36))
 (segment (start 133.54 71.35) (end 139.871 77.681) (width 0.5) (layer "B.Cu") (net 36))
 (segment (start 150.5 84.47) (end 164 97.97) (width 0.5) (layer "B.Cu") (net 36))
 (segment (start 141.859453 81.438635) (end 147.468635 81.438635) (width 0.5) (layer "B.Cu") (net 36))
 (segment (start 139.871 79.450182) (end 141.859453 81.438635) (width 0.5) (layer "B.Cu") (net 36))
 (segment (start 139.871 77.681) (end 139.871 79.450182) (width 0.5) (layer "B.Cu") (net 36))
 (segment (start 147.631374 80.47) (end 151.065687 83.904313) (width 0.5) (layer "F.Cu") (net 37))
 (segment (start 147.5 80.47) (end 147.631374 80.47) (width 0.5) (layer "F.Cu") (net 37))
 (via (at 151.065687 83.904313) (size 0.6) (drill 0.3) (layers "F.Cu" "B.Cu") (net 37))
 (via (at 147.5 80.47) (size 0.6) (drill 0.3) (layers "F.Cu" "B.Cu") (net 37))
 (segment (start 142.411 77.681) (end 142.411 79.450182) (width 0.5) (layer "B.Cu") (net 37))
 (segment (start 143.430818 80.47) (end 147.5 80.47) (width 0.5) (layer "B.Cu") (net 37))
 (segment (start 166.5 99.338626) (end 166.5 99.945) (width 0.5) (layer "B.Cu") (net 37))
 (segment (start 142.411 79.450182) (end 143.430818 80.47) (width 0.5) (layer "B.Cu") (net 37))
 (segment (start 151.065687 83.904313) (end 166.5 99.338626) (width 0.5) (layer "B.Cu") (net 37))
 (segment (start 136.08 71.35) (end 142.411 77.681) (width 0.5) (layer "B.Cu") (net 37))
 (segment (start 160.829 75.179) (end 160.829 83.274) (width 0.5) (layer "B.Cu") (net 40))
 (segment (start 160.829 83.274) (end 164 86.445) (width 0.5) (layer "B.Cu") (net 40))
 (segment (start 157 71.35) (end 160.829 75.179) (width 0.5) (layer "B.Cu") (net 40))
 (segment (start 158.251 75.141) (end 158.251 83.196) (width 0.5) (layer "B.Cu") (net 39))
 (segment (start 158.251 83.196) (end 161.5 86.445) (width 0.5) (layer "B.Cu") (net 39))
 (segment (start 154.46 71.35) (end 158.251 75.141) (width 0.5) (layer "B.Cu") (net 39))
 (segment (start 163.369 75.179) (end 163.369 83.314) (width 0.5) (layer "B.Cu") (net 41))
 (segment (start 163.369 83.314) (end 166.5 86.445) (width 0.5) (layer "B.Cu") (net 41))
 (segment (start 159.54 71.35) (end 163.369 75.179) (width 0.5) (layer "B.Cu") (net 41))
 (segment (start 155.711 75.141) (end 155.711 83.156) (width 0.5) (layer "B.Cu") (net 38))
 (segment (start 155.711 83.156) (end 159 86.445) (width 0.5) (layer "B.Cu") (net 38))
 (segment (start 151.92 71.35) (end 155.711 75.141) (width 0.5) (layer "B.Cu") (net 38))
 (segment (start 143.74 115.78) (end 139.021 111.061) (width 0.2) (layer "F.Cu") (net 21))
 (segment (start 139.021 111.061) (end 139.021 81.109) (width 0.2) (layer "F.Cu") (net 21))
 (segment (start 139.021 81.109) (end 141.16 78.97) (width 0.2) (layer "F.Cu") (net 21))
 (segment (start 151 69.47) (end 152.5 69.47) (width 0.2) (layer "B.Cu") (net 13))
 (segment (start 131.599 114.6539) (end 131.599 98.7239) (width 0.2) (layer "B.Cu") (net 13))
 (segment (start 128.5 123.4) (end 127.399 122.299) (width 0.2) (layer "B.Cu") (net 13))
 (segment (start 150 80.3229) (end 150 70.47) (width 0.2) (layer "B.Cu") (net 13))
 (segment (start 127.399 122.299) (end 127.399 117.86395) (width 0.2) (layer "B.Cu") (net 13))
 (segment (start 152.5 69.47) (end 153.021 69.991) (width 0.2) (layer "B.Cu") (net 13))
 (segment (start 129.0339 117.219) (end 131.599 114.6539) (width 0.2) (layer "B.Cu") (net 13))
 (segment (start 150 70.47) (end 151 69.47) (width 0.2) (layer "B.Cu") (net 13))
 (segment (start 131.599 98.7239) (end 150 80.3229) (width 0.2) (layer "B.Cu") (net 13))
 (segment (start 127.399 117.86395) (end 128.04395 117.219) (width 0.2) (layer "B.Cu") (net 13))
 (segment (start 128.04395 117.219) (end 129.0339 117.219) (width 0.2) (layer "B.Cu") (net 13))
 (segment (start 153.021 71.671768) (end 157 75.650768) (width 0.2) (layer "B.Cu") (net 13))
 (segment (start 153.021 69.991) (end 153.021 71.671768) (width 0.2) (layer "B.Cu") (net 13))
 (segment (start 157 75.650768) (end 157 78.97) (width 0.2) (layer "B.Cu") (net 13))
 (segment (start 143.74 118.32) (end 138.62 113.2) (width 0.2) (layer "F.Cu") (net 20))
 (segment (start 138.62 113.2) (end 138.62 78.97) (width 0.2) (layer "F.Cu") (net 20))
 (segment (start 128.5 120.86) (end 132.401 116.959) (width 0.2) (layer "B.Cu") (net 12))
 (segment (start 132.401 116.959) (end 132.401 101.029) (width 0.2) (layer "B.Cu") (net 12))
 (segment (start 132.401 101.029) (end 154.46 78.97) (width 0.2) (layer "B.Cu") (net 12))
 (segment (start 139.5 83.17) (end 143.7 78.97) (width 0.2) (layer "F.Cu") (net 22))
 (segment (start 139.5 109) (end 139.5 83.17) (width 0.2) (layer "F.Cu") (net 22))
 (segment (start 143.74 113.24) (end 139.5 109) (width 0.2) (layer "F.Cu") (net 22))
 (segment (start 132 98.89) (end 151.92 78.97) (width 0.2) (layer "B.Cu") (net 11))
 (segment (start 128.5 118.32) (end 132 114.82) (width 0.2) (layer "B.Cu") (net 11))
 (segment (start 132 114.82) (end 132 98.89) (width 0.2) (layer "B.Cu") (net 11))
 (segment (start 131.198 114.4878) (end 131.198 98.5578) (width 0.2) (layer "B.Cu") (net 14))
 (segment (start 150.8339 69.069) (end 153.73605 69.069) (width 0.2) (layer "B.Cu") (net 14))
 (segment (start 131.198 98.5578) (end 149.599 80.1568) (width 0.2) (layer "B.Cu") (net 14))
 (segment (start 126.998 115.72495) (end 128.23515 114.4878) (width 0.2) (layer "B.Cu") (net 14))
 (segment (start 149.599 70.3039) (end 150.8339 69.069) (width 0.2) (layer "B.Cu") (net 14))
 (segment (start 126.998 124.438) (end 126.998 115.72495) (width 0.2) (layer "B.Cu") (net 14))
 (segment (start 128.5 125.94) (end 126.998 124.438) (width 0.2) (layer "B.Cu") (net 14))
 (segment (start 155.561 71.671768) (end 159.54 75.650768) (width 0.2) (layer "B.Cu") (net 14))
 (segment (start 128.23515 114.4878) (end 131.198 114.4878) (width 0.2) (layer "B.Cu") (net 14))
 (segment (start 159.54 75.650768) (end 159.54 78.97) (width 0.2) (layer "B.Cu") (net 14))
 (segment (start 149.599 80.1568) (end 149.599 70.3039) (width 0.2) (layer "B.Cu") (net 14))
 (segment (start 153.73605 69.069) (end 155.561 70.89395) (width 0.2) (layer "B.Cu") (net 14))
 (segment (start 155.561 70.89395) (end 155.561 71.671768) (width 0.2) (layer "B.Cu") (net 14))
 (segment (start 143.74 120.86) (end 146 118.6) (width 0.2) (layer "F.Cu") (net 19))
 (segment (start 146 95.05) (end 162.08 78.97) (width 0.2) (layer "F.Cu") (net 19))
 (segment (start 146 118.6) (end 146 95.05) (width 0.2) (layer "F.Cu") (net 19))
 (segment (start 146.24 92.96) (end 146.24 78.97) (width 0.8) (layer "F.Cu") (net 4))
 (segment (start 143.219818 77.719) (end 144.989 77.719) (width 0.5) (layer "F.Cu") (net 4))
 (segment (start 144.989 77.719) (end 146.24 78.97) (width 0.5) (layer "F.Cu") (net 4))
 (segment (start 135 67.97) (end 137.369 70.339) (width 0.5) (layer "F.Cu") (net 4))
 (segment (start 155.5 133.97) (end 147.5 133.97) (width 0.8) (layer "F.Cu") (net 4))
 (segment (start 156.5 126.97) (end 152 131.47) (width 0.8) (layer "F.Cu") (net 4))
 (segment (start 146.24 78.97) (end 147.641 77.569) (width 0.8) (layer "F.Cu") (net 4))
 (segment (start 162.5 126.97) (end 156.5 126.97) (width 0.8) (layer "F.Cu") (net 4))
 (segment (start 143.74 95.46) (end 146.24 92.96) (width 0.8) (layer "F.Cu") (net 4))
 (segment (start 168.299 77.569) (end 169.7 78.97) (width 0.8) (layer "F.Cu") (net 4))
 (segment (start 126 103.04) (end 128.5 100.54) (width 0.8) (layer "F.Cu") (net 4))
 (segment (start 130.254343 133.97) (end 126 129.715657) (width 0.8) (layer "F.Cu") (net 4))
 (segment (start 147.5 126.28) (end 147.5 133.97) (width 0.2) (layer "F.Cu") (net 4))
 (segment (start 147.641 77.569) (end 168.299 77.569) (width 0.8) (layer "F.Cu") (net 4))
 (segment (start 162.5 126.97) (end 155.5 133.97) (width 0.8) (layer "F.Cu") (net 4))
 (segment (start 150.5 123.28) (end 147.5 126.28) (width 0.2) (layer "F.Cu") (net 4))
 (segment (start 147.5 133.97) (end 130.254343 133.97) (width 0.8) (layer "F.Cu") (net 4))
 (segment (start 137.369 70.339) (end 137.369 71.868182) (width 0.5) (layer "F.Cu") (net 4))
 (segment (start 126 129.715657) (end 126 103.04) (width 0.8) (layer "F.Cu") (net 4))
 (segment (start 137.369 71.868182) (end 143.219818 77.719) (width 0.5) (layer "F.Cu") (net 4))
 (segment (start 169.702314 69.371) (end 171.5 71.168686) (width 0.8) (layer "B.Cu") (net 4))
 (segment (start 152 131.47) (end 146.5 125.97) (width 0.8) (layer "B.Cu") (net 4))
 (segment (start 171.5 71.168686) (end 171.5 77.17) (width 0.8) (layer "B.Cu") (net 4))
 (segment (start 171.5 77.17) (end 169.7 78.97) (width 0.8) (layer "B.Cu") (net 4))
 (segment (start 146.5 125.97) (end 146.5 98.22) (width 0.8) (layer "B.Cu") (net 4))
 (segment (start 158.5 67.97) (end 159.901 69.371) (width 0.8) (layer "B.Cu") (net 4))
 (segment (start 159.901 69.371) (end 169.702314 69.371) (width 0.8) (layer "B.Cu") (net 4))
 (segment (start 146.5 98.22) (end 143.74 95.46) (width 0.8) (layer "B.Cu") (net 4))
 (segment (start 150.5 110.51) (end 150.46 110.47) (width 0.2) (layer "F.Cu") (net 42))
 (segment (start 150.5 115.66) (end 150.5 110.51) (width 0.2) (layer "F.Cu") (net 42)))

